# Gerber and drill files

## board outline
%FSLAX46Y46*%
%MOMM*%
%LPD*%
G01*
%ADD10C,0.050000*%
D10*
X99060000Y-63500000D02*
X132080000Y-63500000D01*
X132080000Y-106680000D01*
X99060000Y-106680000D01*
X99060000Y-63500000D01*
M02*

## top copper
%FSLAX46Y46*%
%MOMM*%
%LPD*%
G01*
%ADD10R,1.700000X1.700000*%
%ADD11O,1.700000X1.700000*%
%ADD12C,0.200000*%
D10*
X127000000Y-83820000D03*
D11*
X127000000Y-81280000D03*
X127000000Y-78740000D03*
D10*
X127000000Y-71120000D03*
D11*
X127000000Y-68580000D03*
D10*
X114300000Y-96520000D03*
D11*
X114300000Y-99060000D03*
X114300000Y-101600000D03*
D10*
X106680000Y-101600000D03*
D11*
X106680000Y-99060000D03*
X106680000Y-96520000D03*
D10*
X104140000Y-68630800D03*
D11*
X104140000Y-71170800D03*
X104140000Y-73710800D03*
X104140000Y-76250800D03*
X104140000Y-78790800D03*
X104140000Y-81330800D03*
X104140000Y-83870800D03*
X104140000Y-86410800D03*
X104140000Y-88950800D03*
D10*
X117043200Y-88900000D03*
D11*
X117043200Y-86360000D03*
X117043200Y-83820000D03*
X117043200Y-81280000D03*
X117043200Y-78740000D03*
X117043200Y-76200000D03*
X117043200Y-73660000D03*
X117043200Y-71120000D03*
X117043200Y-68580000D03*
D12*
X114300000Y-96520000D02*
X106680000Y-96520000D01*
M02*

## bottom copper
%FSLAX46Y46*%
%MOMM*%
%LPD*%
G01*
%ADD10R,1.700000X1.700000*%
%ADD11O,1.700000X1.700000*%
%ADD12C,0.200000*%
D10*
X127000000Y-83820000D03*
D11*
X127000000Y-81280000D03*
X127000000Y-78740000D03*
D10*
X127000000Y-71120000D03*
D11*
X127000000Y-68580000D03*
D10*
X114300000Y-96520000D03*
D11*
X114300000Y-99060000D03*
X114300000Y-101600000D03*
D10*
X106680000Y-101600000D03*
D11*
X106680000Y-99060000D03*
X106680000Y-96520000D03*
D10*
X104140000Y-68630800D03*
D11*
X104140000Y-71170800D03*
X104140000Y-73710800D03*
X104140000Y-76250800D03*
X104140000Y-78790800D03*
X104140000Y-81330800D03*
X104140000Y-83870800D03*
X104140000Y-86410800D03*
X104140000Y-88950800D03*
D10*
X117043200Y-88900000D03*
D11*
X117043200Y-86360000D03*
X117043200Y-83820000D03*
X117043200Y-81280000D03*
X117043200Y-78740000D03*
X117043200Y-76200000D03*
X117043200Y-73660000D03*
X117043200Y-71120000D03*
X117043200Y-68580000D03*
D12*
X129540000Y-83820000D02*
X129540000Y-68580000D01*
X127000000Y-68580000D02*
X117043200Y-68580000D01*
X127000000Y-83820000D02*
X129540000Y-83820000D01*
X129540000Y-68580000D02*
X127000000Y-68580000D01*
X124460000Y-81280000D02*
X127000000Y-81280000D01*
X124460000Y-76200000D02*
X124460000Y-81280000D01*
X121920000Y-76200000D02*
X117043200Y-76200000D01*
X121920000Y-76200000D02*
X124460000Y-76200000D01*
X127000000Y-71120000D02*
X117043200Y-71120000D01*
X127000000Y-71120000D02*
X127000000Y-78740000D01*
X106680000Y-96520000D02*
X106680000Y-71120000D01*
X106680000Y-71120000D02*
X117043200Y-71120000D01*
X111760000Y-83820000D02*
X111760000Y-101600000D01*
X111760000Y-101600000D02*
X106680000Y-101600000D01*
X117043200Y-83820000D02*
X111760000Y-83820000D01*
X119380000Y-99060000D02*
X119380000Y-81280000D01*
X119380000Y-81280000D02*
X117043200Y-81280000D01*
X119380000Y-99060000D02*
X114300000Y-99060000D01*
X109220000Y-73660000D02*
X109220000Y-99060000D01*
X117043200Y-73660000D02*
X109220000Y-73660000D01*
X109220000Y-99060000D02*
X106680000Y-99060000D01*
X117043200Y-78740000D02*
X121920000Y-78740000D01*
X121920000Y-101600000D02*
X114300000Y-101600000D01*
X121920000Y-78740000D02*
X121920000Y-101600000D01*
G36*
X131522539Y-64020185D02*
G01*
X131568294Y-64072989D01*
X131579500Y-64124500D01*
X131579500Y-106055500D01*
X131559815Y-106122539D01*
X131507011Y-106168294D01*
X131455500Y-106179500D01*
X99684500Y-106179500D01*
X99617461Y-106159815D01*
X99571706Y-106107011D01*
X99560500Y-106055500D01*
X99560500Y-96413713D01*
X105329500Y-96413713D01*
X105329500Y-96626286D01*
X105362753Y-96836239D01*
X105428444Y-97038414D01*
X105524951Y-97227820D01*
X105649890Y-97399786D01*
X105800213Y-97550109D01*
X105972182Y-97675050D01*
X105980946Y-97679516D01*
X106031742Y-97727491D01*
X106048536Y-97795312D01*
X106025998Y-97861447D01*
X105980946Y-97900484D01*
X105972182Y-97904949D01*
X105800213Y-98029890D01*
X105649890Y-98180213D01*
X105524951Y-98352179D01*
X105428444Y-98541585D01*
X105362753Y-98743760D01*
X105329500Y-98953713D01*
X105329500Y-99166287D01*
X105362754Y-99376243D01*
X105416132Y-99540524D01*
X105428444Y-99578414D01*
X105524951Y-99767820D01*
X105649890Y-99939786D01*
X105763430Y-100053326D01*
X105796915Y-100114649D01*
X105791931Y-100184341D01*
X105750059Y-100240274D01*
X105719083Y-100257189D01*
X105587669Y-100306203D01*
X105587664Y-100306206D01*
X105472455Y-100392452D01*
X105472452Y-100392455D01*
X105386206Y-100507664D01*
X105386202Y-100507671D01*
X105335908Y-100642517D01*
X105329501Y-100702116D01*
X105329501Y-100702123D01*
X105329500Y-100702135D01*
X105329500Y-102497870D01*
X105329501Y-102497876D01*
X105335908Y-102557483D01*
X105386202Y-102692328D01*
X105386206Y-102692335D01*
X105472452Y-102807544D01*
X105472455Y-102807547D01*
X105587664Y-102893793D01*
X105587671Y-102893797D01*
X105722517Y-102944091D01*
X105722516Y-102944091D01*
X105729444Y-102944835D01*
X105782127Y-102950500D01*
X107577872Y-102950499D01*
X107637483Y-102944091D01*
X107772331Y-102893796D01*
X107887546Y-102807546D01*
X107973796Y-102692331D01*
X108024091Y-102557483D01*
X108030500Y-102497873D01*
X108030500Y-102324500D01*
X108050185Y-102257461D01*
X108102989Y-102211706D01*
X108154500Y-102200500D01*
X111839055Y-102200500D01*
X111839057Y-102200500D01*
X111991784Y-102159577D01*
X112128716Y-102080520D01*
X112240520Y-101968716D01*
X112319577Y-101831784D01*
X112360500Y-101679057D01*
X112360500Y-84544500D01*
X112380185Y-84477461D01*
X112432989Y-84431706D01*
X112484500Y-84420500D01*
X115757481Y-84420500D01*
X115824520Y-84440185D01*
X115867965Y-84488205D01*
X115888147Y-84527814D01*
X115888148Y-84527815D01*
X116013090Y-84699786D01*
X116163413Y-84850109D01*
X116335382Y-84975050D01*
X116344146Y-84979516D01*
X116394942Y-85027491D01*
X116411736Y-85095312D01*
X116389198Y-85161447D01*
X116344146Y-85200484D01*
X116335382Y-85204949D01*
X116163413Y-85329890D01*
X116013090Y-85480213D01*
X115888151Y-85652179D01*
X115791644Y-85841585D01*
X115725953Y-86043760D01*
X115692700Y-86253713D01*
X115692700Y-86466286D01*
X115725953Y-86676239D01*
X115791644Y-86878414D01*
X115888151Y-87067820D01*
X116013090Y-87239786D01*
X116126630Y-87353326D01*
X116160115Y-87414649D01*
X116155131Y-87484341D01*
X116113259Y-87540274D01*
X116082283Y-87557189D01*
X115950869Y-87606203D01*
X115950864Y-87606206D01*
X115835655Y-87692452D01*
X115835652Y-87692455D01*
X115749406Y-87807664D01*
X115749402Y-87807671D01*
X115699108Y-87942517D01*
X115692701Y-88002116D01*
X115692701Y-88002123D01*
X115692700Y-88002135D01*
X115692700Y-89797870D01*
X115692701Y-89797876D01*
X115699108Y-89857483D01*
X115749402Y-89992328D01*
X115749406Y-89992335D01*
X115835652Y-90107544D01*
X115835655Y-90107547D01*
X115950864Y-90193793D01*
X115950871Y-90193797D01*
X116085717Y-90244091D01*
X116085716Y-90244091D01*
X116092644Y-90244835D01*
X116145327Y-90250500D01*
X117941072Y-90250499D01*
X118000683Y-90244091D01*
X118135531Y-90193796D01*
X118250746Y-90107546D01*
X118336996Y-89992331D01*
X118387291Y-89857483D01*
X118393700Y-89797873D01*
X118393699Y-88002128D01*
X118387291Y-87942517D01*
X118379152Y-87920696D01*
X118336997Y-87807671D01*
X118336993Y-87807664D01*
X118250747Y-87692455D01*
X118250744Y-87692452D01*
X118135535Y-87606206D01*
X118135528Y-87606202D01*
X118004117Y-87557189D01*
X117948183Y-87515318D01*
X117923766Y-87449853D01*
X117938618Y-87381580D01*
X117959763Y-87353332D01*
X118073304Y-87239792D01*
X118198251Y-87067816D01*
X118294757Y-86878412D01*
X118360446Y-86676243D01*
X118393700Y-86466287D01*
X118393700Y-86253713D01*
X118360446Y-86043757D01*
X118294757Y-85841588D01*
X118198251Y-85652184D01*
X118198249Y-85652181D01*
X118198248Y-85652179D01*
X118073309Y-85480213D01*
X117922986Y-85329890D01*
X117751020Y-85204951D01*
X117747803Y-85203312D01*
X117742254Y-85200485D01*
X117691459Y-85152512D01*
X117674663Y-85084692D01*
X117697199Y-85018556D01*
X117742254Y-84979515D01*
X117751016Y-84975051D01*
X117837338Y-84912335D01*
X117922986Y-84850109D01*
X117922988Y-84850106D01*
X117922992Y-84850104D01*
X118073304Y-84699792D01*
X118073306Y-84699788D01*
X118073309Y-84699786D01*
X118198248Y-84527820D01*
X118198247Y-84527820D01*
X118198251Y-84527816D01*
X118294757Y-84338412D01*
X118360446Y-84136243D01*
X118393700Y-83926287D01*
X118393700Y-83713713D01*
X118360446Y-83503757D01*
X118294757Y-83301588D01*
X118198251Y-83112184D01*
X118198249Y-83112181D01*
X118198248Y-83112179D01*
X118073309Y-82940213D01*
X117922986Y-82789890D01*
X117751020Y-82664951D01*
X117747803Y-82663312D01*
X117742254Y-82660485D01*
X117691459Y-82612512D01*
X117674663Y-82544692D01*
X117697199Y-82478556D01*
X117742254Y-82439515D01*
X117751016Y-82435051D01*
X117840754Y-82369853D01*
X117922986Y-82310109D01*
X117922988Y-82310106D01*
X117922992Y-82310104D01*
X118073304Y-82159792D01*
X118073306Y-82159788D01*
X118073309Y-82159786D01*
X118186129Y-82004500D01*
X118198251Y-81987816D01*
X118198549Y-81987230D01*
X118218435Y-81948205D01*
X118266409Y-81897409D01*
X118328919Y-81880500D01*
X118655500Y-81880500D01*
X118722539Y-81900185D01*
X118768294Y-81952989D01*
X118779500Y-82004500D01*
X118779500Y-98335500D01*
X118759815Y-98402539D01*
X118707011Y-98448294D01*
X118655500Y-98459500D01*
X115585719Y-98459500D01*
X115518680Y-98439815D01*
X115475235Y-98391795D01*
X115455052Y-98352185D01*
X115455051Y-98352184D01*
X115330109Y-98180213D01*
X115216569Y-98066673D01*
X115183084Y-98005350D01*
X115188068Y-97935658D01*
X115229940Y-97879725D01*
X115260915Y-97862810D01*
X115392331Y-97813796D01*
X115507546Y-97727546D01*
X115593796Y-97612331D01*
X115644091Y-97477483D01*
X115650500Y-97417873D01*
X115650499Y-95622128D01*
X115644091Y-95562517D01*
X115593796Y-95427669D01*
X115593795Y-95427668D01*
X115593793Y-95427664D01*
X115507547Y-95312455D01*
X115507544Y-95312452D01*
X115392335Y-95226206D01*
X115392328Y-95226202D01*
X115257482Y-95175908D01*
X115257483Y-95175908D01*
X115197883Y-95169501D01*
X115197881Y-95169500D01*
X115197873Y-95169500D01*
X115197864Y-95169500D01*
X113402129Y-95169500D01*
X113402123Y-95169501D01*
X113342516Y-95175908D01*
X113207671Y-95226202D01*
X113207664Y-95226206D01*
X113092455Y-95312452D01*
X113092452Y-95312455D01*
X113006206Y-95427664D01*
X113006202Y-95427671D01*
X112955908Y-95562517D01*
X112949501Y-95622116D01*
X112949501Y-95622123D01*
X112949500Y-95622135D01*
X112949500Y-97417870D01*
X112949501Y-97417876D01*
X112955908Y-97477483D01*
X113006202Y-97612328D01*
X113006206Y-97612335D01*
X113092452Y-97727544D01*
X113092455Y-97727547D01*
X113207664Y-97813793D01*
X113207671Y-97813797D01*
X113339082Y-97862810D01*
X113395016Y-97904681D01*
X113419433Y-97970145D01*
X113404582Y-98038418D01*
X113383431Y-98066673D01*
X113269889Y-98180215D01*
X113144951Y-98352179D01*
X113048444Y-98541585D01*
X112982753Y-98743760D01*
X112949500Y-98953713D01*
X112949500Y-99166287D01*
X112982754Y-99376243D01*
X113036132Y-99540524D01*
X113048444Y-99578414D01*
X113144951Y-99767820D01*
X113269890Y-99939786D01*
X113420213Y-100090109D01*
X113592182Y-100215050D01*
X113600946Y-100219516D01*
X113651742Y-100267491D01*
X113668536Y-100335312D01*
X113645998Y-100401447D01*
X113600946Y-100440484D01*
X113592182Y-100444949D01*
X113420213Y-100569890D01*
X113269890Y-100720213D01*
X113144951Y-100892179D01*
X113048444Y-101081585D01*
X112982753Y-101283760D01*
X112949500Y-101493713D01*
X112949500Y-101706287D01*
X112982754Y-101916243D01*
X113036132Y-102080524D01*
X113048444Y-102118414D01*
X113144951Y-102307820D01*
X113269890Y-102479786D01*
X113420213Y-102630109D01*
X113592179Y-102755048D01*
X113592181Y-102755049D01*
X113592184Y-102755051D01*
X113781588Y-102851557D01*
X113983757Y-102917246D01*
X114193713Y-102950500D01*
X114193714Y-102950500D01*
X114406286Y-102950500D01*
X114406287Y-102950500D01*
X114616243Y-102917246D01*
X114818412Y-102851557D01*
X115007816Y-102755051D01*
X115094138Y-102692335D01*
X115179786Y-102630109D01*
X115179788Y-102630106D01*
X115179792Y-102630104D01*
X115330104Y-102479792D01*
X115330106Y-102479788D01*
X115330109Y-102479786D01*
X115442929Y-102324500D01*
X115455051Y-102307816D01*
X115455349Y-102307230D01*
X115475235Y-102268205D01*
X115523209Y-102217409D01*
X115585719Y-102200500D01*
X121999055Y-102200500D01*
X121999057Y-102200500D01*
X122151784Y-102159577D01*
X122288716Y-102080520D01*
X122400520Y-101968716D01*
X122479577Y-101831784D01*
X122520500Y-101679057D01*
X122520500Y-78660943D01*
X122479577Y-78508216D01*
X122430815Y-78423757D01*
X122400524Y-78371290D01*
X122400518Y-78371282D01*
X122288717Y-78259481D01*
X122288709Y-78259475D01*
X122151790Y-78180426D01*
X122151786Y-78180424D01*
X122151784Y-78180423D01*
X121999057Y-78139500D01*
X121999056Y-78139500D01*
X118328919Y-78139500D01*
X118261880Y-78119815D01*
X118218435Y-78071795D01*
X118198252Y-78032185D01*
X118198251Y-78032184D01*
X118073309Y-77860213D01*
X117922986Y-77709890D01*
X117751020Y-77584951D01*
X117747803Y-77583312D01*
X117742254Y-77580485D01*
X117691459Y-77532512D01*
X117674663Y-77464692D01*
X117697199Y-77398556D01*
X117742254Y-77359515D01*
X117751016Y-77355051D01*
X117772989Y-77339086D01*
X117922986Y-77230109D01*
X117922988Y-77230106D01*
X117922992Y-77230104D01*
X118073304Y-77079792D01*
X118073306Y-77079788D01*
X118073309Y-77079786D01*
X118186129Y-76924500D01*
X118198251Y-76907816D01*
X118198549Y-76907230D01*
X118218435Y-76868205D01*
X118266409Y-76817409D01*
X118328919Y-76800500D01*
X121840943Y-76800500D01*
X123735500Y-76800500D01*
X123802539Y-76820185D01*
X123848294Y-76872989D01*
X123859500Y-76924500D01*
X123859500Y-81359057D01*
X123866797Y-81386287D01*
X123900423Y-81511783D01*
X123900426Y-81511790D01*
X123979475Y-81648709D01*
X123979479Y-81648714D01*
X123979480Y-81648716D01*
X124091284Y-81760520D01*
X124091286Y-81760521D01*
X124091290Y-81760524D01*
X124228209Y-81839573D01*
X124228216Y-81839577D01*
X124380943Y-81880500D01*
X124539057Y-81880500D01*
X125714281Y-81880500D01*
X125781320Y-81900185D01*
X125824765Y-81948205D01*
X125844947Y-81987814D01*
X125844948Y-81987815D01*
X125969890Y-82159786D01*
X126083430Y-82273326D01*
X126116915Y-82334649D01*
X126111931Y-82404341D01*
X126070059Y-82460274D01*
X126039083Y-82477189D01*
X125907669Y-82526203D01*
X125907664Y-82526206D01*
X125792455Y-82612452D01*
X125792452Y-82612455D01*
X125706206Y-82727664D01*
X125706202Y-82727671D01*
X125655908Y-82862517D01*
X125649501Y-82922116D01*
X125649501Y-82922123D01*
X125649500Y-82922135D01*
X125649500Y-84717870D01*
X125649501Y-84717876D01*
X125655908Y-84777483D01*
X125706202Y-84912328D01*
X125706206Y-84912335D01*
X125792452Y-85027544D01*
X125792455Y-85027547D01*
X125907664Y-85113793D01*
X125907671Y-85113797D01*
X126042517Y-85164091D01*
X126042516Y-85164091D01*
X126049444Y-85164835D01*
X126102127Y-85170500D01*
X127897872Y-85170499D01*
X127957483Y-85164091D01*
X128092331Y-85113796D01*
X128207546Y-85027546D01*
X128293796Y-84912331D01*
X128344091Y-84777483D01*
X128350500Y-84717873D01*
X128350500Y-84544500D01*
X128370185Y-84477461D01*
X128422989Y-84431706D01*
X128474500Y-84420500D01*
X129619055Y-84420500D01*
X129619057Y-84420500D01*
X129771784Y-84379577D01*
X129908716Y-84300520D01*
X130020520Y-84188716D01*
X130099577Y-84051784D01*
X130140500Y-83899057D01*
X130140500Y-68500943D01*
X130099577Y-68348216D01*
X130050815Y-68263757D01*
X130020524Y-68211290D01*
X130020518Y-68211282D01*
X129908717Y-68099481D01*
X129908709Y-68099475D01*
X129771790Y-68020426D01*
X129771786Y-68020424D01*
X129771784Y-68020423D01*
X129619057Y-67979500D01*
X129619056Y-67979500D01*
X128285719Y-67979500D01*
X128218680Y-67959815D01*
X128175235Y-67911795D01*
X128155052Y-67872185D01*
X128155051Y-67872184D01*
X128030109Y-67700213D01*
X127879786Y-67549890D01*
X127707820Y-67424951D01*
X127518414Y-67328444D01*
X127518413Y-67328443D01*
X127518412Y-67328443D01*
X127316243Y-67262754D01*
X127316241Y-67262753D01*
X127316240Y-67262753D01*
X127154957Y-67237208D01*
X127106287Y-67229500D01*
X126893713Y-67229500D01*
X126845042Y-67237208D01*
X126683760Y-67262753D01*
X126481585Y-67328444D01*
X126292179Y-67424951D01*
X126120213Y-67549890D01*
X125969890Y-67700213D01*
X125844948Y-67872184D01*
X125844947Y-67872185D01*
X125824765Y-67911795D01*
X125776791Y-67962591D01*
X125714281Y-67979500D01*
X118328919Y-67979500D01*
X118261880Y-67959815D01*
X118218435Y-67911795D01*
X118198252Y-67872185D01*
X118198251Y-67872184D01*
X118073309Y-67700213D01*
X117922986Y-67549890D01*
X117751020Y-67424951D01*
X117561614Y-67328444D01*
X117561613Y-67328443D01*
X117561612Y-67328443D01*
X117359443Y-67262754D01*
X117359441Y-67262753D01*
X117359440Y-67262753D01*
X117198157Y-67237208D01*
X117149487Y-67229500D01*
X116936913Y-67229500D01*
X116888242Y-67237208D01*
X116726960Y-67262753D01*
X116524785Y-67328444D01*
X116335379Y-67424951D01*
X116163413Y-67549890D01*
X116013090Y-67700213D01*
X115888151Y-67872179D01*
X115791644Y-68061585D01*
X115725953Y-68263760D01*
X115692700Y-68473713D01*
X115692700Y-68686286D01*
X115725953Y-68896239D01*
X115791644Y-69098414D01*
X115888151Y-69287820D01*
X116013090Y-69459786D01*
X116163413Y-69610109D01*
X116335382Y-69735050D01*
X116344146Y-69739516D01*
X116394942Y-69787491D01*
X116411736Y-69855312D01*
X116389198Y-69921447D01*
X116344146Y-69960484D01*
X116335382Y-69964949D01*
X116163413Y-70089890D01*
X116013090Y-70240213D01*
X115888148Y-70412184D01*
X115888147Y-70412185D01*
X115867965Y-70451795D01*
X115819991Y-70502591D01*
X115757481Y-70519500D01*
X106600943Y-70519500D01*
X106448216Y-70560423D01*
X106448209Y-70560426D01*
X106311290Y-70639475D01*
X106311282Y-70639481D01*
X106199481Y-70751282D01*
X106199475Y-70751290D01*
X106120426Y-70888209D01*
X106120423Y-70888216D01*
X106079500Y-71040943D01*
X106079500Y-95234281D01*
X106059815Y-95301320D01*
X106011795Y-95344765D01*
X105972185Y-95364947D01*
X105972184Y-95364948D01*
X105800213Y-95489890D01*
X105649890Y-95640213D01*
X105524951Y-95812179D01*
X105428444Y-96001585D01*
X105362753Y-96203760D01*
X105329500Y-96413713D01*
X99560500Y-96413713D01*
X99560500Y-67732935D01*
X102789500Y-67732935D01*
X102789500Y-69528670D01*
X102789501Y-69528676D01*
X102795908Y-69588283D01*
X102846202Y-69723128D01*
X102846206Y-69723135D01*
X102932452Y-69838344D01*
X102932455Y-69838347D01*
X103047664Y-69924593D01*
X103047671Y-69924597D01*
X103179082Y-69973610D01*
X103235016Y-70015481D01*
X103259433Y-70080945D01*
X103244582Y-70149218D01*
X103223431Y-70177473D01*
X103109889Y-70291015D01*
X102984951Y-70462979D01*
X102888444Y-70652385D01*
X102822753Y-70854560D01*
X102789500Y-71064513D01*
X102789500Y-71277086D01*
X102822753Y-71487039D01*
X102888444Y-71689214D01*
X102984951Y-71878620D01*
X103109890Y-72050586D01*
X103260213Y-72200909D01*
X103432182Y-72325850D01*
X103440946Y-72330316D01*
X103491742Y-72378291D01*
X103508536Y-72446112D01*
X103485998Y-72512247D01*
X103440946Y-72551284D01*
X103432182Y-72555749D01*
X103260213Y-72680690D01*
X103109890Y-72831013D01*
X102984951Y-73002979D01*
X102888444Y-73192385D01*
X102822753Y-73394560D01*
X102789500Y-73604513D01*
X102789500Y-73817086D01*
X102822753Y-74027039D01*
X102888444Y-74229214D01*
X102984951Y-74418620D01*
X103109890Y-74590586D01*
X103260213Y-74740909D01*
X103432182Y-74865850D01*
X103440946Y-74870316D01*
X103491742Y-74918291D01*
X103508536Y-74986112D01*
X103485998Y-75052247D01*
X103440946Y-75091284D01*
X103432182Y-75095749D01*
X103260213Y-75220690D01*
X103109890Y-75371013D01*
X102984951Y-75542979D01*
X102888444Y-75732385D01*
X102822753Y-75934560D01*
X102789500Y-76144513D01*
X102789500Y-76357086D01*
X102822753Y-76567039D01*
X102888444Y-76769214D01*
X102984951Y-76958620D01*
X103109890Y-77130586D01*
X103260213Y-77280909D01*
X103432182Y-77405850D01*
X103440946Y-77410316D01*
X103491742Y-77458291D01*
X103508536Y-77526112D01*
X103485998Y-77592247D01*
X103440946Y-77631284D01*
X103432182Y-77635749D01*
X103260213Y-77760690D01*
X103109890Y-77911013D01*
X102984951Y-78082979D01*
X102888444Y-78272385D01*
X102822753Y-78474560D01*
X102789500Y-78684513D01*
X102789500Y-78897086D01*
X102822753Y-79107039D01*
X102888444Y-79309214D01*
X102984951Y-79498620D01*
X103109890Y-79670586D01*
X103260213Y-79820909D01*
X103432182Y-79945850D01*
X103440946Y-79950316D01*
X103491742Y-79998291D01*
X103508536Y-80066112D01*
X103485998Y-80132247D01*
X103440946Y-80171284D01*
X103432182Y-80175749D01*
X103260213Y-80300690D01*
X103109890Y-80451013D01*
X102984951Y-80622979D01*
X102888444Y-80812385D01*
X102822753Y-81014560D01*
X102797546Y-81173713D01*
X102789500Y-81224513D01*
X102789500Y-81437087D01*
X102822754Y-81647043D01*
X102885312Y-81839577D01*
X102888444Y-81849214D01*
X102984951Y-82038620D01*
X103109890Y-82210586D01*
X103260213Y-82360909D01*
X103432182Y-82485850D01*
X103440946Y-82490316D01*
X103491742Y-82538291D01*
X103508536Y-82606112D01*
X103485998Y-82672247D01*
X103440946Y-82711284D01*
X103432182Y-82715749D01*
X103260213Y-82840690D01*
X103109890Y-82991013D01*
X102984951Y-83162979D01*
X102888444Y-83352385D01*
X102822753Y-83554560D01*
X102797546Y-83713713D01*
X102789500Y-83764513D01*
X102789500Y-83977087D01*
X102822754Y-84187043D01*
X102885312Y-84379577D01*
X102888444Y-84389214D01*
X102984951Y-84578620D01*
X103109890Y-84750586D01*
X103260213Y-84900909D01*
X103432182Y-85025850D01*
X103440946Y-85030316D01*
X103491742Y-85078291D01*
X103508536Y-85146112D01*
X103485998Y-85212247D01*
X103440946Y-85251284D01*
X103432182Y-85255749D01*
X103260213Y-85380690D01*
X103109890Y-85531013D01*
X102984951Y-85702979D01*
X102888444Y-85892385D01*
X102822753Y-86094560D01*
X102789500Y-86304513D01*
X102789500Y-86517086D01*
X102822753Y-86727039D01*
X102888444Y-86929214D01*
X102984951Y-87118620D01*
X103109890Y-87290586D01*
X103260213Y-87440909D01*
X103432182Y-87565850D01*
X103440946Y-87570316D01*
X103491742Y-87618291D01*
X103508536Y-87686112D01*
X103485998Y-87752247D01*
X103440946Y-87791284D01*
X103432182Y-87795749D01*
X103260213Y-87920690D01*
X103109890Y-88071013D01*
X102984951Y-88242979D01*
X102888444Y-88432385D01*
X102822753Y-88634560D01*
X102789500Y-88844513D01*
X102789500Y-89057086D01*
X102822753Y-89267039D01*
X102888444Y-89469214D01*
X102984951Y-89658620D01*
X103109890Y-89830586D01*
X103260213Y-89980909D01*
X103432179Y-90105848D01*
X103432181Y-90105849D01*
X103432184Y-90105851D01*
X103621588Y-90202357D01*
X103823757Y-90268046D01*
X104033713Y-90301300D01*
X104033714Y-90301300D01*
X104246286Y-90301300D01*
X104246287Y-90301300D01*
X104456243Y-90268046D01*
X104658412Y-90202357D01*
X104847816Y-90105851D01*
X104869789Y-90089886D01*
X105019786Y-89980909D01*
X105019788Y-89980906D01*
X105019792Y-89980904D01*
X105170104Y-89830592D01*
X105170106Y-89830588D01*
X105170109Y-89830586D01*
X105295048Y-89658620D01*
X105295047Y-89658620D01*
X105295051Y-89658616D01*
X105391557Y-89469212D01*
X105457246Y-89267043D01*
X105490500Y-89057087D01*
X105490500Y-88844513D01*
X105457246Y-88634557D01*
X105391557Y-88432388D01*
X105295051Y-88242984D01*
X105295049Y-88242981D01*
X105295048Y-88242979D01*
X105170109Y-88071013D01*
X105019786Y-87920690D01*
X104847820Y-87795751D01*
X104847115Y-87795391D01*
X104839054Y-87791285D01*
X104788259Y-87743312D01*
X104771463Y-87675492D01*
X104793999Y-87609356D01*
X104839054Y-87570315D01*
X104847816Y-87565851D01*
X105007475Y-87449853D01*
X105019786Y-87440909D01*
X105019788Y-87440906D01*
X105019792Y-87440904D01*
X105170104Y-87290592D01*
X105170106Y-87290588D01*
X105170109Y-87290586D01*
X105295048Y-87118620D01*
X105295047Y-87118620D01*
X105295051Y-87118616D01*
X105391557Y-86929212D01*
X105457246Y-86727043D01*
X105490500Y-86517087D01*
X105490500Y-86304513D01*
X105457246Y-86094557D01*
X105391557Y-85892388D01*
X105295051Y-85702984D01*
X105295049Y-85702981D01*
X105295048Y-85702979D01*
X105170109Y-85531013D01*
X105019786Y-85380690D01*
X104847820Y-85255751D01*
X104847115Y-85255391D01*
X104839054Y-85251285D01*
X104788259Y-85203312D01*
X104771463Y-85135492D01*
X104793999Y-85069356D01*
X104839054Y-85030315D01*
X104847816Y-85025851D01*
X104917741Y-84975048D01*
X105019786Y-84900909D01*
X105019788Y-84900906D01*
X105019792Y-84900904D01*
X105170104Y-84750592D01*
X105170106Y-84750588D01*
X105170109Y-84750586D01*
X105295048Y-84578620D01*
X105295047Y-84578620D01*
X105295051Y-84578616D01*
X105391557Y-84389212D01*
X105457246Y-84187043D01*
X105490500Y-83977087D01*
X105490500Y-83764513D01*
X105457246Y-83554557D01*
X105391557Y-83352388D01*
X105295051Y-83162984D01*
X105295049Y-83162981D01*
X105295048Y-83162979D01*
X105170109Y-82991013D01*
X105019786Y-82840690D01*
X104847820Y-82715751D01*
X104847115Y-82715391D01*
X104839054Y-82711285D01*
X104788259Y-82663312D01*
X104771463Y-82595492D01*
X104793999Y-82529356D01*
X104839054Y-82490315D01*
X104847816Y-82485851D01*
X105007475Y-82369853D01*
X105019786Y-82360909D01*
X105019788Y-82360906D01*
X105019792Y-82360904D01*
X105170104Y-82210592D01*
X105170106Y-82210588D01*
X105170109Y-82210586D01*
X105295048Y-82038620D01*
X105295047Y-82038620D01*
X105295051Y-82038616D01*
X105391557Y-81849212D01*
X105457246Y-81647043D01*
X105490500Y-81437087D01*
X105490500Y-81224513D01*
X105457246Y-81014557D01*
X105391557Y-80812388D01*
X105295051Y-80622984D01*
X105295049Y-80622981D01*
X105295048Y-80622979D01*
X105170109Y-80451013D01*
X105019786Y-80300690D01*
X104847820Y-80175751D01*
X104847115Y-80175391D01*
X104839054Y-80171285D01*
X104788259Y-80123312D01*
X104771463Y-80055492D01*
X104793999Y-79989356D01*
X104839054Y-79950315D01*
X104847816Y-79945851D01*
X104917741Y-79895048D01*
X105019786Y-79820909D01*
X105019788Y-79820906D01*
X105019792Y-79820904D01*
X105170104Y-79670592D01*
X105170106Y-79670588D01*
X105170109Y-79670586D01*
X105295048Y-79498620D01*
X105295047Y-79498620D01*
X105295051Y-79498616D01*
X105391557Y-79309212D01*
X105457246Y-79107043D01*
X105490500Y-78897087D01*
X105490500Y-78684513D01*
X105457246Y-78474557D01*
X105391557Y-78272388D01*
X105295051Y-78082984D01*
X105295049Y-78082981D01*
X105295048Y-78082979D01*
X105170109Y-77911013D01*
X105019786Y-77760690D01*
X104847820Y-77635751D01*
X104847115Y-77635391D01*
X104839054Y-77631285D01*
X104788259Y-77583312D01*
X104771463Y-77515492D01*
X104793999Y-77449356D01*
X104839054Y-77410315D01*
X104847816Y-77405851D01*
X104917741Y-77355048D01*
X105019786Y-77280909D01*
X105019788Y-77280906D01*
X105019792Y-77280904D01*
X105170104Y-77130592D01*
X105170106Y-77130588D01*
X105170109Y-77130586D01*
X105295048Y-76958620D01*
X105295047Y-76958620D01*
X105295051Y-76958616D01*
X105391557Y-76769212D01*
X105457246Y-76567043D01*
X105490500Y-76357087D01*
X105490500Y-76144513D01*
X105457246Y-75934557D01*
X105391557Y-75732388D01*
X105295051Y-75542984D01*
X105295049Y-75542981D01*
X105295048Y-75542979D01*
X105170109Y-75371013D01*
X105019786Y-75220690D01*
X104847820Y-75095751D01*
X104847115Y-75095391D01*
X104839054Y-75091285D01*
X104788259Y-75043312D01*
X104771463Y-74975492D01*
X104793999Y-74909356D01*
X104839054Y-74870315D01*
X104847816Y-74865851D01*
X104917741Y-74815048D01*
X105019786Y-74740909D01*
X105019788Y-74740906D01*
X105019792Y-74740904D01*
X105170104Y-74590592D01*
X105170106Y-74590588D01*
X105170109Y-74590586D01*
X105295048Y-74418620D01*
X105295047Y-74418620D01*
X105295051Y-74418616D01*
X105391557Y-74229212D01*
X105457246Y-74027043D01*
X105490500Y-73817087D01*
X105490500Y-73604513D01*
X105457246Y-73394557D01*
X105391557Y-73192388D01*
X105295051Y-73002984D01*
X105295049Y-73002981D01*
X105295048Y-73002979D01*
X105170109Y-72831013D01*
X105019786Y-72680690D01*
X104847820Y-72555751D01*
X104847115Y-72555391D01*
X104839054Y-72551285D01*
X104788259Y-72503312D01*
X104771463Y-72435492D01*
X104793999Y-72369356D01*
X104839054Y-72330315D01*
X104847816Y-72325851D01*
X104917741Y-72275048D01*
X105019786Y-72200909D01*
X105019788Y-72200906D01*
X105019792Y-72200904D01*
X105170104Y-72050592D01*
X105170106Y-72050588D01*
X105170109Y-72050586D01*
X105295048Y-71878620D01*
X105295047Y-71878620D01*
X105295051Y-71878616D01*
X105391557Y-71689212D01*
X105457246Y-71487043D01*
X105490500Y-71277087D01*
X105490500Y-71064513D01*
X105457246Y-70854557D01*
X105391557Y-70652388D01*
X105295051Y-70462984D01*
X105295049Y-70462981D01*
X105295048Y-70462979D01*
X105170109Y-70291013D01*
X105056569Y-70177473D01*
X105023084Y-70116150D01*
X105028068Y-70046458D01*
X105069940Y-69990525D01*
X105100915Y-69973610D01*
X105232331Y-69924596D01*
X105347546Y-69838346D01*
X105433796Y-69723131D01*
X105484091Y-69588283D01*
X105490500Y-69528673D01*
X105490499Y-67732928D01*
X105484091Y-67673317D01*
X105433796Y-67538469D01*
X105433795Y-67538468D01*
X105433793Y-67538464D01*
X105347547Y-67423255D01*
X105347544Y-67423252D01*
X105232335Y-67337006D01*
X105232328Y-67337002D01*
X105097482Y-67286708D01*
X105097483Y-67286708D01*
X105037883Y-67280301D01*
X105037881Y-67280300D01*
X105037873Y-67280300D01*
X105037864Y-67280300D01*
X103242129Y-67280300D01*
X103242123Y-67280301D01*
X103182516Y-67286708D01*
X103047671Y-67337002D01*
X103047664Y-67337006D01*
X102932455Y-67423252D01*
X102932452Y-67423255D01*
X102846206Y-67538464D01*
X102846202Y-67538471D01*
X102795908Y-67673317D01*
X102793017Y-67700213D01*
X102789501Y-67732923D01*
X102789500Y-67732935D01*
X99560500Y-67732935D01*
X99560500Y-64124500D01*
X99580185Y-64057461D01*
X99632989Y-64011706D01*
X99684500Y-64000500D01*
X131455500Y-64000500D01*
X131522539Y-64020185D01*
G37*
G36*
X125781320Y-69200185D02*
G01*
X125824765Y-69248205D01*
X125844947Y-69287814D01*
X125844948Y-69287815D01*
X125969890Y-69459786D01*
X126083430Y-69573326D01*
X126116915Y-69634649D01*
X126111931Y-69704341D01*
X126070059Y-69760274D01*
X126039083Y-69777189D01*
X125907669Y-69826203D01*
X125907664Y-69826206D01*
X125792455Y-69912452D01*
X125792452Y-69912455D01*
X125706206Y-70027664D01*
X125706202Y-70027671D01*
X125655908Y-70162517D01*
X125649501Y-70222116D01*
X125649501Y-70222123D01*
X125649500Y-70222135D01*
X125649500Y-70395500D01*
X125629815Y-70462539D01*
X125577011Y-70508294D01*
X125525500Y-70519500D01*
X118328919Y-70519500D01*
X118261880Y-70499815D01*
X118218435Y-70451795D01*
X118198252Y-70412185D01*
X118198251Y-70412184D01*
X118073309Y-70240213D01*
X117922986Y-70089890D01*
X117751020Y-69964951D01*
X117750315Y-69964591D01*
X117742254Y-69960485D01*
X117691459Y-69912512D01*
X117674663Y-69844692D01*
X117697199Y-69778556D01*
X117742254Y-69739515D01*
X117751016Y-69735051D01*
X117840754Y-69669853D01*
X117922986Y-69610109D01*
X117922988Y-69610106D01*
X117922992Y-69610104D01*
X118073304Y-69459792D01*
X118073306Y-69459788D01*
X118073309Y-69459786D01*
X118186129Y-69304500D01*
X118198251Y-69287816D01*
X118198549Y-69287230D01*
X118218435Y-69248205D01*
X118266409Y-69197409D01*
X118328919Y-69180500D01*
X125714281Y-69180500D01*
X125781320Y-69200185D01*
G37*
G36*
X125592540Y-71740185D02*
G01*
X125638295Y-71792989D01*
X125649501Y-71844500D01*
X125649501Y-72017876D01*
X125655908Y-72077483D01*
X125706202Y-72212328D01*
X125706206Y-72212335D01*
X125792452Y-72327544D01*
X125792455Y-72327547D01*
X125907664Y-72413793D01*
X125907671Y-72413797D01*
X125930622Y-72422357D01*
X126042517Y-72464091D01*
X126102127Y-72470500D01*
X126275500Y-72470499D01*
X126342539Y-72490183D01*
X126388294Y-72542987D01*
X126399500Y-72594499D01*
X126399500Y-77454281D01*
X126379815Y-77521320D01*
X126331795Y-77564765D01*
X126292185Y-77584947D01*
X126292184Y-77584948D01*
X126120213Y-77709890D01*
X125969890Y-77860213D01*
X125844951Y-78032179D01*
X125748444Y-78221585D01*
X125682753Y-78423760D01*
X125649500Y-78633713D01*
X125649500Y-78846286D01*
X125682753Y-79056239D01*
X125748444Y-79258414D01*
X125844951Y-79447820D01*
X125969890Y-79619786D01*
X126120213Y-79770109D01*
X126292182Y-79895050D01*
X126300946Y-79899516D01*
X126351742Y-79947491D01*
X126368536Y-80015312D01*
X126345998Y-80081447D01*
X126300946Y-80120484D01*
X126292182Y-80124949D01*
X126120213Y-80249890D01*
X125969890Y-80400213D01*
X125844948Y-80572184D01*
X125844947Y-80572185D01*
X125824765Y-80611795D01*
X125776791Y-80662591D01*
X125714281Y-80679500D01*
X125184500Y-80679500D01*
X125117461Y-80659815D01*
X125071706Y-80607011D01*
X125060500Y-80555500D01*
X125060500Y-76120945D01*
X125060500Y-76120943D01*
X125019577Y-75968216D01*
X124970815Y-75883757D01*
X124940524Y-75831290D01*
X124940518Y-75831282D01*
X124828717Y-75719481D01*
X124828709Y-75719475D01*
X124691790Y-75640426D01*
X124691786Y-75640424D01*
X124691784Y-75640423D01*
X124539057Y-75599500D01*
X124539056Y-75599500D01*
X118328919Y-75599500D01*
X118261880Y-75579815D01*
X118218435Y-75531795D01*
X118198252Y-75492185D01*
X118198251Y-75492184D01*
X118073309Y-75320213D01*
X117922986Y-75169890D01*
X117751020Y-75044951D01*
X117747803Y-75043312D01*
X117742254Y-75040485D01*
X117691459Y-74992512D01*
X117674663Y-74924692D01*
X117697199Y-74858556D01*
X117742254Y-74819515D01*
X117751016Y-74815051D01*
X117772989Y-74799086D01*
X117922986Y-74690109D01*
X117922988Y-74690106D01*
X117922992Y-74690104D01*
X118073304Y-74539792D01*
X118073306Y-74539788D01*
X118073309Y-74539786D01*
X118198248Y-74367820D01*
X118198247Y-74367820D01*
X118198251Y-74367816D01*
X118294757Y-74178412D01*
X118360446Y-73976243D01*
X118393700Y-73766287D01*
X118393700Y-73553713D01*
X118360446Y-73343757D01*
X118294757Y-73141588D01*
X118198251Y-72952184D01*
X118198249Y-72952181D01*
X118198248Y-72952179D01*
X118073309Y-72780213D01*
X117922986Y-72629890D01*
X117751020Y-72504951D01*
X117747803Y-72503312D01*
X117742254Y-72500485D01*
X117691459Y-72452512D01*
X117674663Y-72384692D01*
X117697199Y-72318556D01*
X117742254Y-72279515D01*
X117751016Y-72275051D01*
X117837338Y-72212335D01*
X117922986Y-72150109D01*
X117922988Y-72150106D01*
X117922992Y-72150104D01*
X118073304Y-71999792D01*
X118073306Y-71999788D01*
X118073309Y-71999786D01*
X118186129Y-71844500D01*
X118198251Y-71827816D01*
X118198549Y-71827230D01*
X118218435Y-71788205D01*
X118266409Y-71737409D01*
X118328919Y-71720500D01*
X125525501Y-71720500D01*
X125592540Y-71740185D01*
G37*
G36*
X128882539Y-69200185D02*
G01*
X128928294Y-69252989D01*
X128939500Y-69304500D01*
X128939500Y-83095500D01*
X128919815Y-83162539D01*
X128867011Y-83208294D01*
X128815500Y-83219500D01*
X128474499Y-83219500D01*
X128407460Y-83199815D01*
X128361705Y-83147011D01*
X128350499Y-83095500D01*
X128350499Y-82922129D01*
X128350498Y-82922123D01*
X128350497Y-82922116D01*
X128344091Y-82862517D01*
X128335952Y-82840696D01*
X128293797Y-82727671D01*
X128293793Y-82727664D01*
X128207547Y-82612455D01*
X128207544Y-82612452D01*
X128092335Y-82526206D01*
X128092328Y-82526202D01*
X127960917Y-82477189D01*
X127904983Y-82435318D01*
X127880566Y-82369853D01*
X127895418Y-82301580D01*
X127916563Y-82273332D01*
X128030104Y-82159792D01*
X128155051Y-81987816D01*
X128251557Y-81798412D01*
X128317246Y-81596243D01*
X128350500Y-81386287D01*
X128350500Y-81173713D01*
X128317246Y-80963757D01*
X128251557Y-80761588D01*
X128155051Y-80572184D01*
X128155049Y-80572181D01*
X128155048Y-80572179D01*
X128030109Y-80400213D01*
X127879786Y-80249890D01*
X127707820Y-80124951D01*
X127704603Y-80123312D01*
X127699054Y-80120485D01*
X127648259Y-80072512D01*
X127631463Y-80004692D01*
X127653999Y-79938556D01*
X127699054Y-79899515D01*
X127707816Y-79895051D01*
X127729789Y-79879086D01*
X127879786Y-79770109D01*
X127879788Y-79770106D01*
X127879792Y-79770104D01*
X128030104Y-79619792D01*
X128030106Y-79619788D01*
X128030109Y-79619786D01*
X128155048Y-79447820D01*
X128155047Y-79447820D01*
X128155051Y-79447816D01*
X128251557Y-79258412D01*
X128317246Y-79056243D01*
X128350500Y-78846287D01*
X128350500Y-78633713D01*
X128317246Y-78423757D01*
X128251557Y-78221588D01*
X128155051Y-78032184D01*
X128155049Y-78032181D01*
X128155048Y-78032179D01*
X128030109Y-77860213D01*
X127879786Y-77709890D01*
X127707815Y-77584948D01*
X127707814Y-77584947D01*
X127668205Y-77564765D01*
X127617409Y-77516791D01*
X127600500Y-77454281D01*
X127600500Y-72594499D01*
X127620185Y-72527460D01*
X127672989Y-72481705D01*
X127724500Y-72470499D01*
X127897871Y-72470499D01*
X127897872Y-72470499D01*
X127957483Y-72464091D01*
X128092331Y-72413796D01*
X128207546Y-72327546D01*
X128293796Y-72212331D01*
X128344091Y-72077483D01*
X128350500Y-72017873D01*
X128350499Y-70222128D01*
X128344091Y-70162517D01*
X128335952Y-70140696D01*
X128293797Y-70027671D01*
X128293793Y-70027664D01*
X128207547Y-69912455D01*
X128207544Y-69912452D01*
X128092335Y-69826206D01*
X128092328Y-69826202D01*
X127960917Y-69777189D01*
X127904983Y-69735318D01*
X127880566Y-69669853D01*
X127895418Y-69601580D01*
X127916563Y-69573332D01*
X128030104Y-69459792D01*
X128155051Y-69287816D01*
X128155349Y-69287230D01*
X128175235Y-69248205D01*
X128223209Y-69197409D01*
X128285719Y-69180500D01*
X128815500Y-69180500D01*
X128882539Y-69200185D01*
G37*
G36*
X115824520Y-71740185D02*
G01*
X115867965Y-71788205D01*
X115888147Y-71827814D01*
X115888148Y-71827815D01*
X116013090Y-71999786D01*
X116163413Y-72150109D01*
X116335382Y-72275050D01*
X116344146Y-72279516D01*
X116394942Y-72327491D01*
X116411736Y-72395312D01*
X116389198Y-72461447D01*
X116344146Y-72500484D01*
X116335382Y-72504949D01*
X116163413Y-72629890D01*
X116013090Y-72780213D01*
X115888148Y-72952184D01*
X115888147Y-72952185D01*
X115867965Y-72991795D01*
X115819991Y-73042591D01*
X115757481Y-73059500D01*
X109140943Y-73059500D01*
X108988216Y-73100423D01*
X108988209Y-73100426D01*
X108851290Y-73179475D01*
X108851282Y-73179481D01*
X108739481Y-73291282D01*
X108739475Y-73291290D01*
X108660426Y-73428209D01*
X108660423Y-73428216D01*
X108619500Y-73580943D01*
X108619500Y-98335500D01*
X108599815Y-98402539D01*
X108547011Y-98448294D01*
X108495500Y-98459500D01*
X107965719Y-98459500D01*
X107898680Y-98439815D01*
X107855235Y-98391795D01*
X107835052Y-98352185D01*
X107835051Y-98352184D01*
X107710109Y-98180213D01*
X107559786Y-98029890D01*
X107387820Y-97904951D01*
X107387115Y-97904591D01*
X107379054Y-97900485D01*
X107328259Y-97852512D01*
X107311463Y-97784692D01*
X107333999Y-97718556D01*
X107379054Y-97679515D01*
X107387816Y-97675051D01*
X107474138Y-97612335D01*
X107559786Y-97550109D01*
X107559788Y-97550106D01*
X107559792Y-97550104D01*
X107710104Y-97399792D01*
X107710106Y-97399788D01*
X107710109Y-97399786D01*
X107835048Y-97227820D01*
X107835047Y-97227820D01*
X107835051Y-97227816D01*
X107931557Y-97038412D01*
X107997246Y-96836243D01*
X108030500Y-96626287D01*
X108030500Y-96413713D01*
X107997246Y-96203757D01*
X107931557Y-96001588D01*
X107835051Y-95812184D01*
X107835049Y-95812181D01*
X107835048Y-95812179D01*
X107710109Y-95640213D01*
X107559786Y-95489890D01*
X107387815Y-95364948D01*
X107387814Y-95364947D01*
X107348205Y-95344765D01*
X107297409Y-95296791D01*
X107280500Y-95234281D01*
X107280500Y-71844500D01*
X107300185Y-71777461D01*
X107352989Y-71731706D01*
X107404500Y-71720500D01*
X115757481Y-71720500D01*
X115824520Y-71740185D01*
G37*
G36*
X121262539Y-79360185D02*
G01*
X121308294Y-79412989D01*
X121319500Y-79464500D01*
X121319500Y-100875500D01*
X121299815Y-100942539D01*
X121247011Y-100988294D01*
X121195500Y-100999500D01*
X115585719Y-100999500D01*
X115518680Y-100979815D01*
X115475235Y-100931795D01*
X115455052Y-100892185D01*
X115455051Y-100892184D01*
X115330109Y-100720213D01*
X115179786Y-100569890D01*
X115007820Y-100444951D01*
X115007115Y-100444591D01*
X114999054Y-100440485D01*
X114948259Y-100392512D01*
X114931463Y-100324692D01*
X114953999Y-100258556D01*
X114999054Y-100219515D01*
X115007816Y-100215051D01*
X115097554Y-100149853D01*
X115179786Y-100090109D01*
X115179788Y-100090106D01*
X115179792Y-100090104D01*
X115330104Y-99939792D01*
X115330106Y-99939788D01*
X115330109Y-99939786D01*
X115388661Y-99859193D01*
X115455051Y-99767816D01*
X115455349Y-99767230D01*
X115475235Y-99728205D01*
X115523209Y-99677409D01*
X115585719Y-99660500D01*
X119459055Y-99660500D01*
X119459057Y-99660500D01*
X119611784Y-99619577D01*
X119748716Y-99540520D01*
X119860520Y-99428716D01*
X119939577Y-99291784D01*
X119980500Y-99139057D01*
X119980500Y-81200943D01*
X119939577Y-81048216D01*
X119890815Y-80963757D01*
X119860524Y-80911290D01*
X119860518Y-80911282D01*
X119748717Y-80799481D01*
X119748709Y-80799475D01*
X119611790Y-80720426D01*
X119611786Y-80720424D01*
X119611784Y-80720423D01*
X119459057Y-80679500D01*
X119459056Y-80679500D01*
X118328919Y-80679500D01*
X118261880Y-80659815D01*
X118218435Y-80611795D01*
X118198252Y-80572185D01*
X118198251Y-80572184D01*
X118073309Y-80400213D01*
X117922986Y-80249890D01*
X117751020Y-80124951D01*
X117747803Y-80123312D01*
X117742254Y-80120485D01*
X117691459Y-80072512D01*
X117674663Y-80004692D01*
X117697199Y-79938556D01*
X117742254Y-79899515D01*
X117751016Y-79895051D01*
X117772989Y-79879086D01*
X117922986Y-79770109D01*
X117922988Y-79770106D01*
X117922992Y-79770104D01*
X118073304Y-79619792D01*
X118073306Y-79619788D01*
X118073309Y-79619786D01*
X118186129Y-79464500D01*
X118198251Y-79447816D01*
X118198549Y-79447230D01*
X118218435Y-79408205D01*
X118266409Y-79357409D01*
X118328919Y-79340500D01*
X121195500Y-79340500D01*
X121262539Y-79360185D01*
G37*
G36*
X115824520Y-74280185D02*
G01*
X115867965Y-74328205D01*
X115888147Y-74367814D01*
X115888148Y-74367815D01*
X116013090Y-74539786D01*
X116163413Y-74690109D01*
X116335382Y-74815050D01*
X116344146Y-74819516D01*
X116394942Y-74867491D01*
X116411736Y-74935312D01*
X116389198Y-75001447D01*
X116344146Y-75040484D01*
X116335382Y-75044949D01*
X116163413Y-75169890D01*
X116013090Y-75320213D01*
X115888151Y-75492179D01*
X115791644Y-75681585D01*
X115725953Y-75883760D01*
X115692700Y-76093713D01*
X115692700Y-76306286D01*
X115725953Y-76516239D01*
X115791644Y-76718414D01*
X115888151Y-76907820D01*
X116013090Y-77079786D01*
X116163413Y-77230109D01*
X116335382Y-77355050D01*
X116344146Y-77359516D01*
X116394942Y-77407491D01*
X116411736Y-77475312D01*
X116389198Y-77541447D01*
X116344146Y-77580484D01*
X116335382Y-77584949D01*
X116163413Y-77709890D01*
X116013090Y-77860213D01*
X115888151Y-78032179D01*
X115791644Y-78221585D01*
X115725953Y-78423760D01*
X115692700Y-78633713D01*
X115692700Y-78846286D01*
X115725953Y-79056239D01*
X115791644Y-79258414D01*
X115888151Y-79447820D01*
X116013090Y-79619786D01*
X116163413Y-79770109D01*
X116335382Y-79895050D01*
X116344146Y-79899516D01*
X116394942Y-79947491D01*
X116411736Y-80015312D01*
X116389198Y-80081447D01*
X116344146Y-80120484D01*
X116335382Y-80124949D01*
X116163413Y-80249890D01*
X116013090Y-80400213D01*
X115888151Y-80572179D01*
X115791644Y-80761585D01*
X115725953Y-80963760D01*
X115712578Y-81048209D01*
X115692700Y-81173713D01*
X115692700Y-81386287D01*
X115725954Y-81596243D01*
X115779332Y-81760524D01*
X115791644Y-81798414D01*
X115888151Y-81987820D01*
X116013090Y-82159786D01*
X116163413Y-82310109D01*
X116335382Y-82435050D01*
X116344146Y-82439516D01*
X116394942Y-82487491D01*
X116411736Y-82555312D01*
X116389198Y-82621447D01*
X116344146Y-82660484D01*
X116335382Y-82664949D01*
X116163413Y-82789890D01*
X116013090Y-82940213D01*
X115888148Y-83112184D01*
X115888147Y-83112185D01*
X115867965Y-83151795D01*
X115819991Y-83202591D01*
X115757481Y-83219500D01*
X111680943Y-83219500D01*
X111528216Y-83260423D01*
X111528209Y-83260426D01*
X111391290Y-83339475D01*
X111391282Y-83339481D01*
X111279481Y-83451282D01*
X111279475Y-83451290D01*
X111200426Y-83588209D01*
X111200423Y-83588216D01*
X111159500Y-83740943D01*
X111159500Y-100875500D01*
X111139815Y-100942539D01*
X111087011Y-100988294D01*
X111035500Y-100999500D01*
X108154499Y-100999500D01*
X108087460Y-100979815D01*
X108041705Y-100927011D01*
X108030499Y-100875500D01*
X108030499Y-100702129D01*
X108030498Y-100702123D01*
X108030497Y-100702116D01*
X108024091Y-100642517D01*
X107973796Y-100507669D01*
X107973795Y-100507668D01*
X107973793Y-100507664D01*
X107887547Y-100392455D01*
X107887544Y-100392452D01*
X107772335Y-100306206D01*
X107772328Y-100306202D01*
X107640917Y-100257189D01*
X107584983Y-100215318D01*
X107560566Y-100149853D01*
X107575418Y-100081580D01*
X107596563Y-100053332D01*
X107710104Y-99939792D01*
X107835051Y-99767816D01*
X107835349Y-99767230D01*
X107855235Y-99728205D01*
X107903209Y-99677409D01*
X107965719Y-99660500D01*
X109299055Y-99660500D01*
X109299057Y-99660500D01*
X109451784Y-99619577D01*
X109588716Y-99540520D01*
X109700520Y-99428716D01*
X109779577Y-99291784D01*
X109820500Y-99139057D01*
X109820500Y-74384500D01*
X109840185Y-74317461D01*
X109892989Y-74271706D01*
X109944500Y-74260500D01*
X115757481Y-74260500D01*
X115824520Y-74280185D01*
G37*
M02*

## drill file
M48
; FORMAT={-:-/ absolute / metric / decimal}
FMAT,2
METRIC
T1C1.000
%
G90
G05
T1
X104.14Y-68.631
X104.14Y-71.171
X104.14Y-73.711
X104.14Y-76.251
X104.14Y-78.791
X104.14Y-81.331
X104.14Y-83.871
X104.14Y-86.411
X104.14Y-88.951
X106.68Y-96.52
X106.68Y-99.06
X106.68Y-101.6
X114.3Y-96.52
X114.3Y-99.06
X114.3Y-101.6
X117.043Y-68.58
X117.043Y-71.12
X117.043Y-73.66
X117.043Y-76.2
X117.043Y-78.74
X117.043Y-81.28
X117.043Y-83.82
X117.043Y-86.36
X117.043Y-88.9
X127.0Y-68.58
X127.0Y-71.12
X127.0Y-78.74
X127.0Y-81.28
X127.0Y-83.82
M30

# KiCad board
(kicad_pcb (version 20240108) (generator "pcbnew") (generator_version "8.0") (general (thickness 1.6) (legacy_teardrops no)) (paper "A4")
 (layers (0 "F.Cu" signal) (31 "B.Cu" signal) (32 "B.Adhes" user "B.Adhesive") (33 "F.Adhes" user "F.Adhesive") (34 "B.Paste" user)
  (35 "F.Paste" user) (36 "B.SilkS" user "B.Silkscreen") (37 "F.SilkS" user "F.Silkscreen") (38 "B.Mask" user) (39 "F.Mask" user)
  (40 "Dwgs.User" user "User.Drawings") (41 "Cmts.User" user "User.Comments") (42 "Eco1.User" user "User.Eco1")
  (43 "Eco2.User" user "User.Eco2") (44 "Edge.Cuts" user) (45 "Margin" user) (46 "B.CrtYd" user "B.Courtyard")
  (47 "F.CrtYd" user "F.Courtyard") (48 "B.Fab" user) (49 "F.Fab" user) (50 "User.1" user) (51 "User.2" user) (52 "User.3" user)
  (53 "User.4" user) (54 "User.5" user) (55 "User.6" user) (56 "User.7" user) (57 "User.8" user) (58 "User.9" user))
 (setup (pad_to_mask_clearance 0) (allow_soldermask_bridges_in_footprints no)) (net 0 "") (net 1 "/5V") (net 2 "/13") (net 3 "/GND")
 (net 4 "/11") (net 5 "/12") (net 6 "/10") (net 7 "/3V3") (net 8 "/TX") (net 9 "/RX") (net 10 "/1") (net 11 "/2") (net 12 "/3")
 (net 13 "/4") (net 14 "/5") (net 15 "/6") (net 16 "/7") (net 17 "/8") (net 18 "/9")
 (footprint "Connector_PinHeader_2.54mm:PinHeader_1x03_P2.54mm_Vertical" (layer "F.Cu") (at 127 83.82 180)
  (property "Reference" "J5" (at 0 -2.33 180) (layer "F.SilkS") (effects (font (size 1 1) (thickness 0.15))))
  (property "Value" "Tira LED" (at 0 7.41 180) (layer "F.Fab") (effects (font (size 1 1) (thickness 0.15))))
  (pad "1" thru_hole rect (at 0 0 180) (size 1.7 1.7) (drill 1) (layers "*.Cu" "*.Mask") (remove_unused_layers no) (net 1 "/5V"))
  (pad "2" thru_hole oval (at 0 2.54 180) (size 1.7 1.7) (drill 1) (layers "*.Cu" "*.Mask") (remove_unused_layers no) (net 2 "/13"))
  (pad "3" thru_hole oval (at 0 5.08 180) (size 1.7 1.7) (drill 1) (layers "*.Cu" "*.Mask") (remove_unused_layers no) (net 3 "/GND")))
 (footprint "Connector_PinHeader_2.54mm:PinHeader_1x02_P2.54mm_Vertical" (layer "F.Cu") (at 127 71.12 180)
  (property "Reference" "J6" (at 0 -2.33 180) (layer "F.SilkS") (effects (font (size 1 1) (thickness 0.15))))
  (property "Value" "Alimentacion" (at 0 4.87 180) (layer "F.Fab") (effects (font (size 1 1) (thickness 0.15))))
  (pad "1" thru_hole rect (at 0 0 180) (size 1.7 1.7) (drill 1) (layers "*.Cu" "*.Mask") (remove_unused_layers no) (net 3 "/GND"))
  (pad "2" thru_hole oval (at 0 2.54 180) (size 1.7 1.7) (drill 1) (layers "*.Cu" "*.Mask") (remove_unused_layers no) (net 1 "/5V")))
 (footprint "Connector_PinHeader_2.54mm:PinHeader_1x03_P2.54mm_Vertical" (layer "F.Cu") (at 114.3 96.52)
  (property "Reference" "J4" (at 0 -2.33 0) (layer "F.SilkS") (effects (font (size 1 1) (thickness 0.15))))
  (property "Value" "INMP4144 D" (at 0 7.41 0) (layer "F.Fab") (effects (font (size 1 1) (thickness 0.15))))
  (pad "1" thru_hole rect (at 0 0) (size 1.7 1.7) (drill 1) (layers "*.Cu" "*.Mask") (remove_unused_layers no) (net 3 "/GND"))
  (pad "2" thru_hole oval (at 0 2.54) (size 1.7 1.7) (drill 1) (layers "*.Cu" "*.Mask") (remove_unused_layers no) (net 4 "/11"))
  (pad "3" thru_hole oval (at 0 5.08) (size 1.7 1.7) (drill 1) (layers "*.Cu" "*.Mask") (remove_unused_layers no) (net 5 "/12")))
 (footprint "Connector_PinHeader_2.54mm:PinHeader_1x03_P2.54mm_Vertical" (layer "F.Cu") (at 106.68 101.6 180)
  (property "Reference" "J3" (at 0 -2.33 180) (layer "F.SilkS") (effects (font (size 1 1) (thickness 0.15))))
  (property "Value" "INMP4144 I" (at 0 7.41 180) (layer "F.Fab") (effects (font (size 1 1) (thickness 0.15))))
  (pad "1" thru_hole rect (at 0 0 180) (size 1.7 1.7) (drill 1) (layers "*.Cu" "*.Mask") (remove_unused_layers no) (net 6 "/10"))
  (pad "2" thru_hole oval (at 0 2.54 180) (size 1.7 1.7) (drill 1) (layers "*.Cu" "*.Mask") (remove_unused_layers no) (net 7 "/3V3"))
  (pad "3" thru_hole oval (at 0 5.08 180) (size 1.7 1.7) (drill 1) (layers "*.Cu" "*.Mask") (remove_unused_layers no) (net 3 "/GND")))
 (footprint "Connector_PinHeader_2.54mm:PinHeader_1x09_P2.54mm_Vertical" (layer "F.Cu") (at 104.14 68.6308)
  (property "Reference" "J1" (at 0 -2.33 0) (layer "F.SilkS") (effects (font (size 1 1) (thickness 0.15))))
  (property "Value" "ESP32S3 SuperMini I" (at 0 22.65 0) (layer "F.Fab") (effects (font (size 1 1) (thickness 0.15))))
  (pad "1" thru_hole rect (at 0 0) (size 1.7 1.7) (drill 1) (layers "*.Cu" "*.Mask") (remove_unused_layers no) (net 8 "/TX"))
  (pad "2" thru_hole oval (at 0 2.54) (size 1.7 1.7) (drill 1) (layers "*.Cu" "*.Mask") (remove_unused_layers no) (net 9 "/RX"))
  (pad "3" thru_hole oval (at 0 5.08) (size 1.7 1.7) (drill 1) (layers "*.Cu" "*.Mask") (remove_unused_layers no) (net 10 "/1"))
  (pad "4" thru_hole oval (at 0 7.62) (size 1.7 1.7) (drill 1) (layers "*.Cu" "*.Mask") (remove_unused_layers no) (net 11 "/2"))
  (pad "5" thru_hole oval (at 0 10.16) (size 1.7 1.7) (drill 1) (layers "*.Cu" "*.Mask") (remove_unused_layers no) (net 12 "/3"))
  (pad "6" thru_hole oval (at 0 12.7) (size 1.7 1.7) (drill 1) (layers "*.Cu" "*.Mask") (remove_unused_layers no) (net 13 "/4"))
  (pad "7" thru_hole oval (at 0 15.24) (size 1.7 1.7) (drill 1) (layers "*.Cu" "*.Mask") (remove_unused_layers no) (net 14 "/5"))
  (pad "8" thru_hole oval (at 0 17.78) (size 1.7 1.7) (drill 1) (layers "*.Cu" "*.Mask") (remove_unused_layers no) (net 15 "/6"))
  (pad "9" thru_hole oval (at 0 20.32) (size 1.7 1.7) (drill 1) (layers "*.Cu" "*.Mask") (remove_unused_layers no) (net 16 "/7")))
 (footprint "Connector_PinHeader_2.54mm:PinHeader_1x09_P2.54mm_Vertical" (layer "F.Cu") (at 117.0432 88.9 180)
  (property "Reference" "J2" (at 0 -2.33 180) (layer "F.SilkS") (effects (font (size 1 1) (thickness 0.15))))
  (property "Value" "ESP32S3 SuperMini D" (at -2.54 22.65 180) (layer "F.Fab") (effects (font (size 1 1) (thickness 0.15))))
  (pad "1" thru_hole rect (at 0 0 180) (size 1.7 1.7) (drill 1) (layers "*.Cu" "*.Mask") (remove_unused_layers no) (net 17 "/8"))
  (pad "2" thru_hole oval (at 0 2.54 180) (size 1.7 1.7) (drill 1) (layers "*.Cu" "*.Mask") (remove_unused_layers no) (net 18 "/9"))
  (pad "3" thru_hole oval (at 0 5.08 180) (size 1.7 1.7) (drill 1) (layers "*.Cu" "*.Mask") (remove_unused_layers no) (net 6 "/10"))
  (pad "4" thru_hole oval (at 0 7.62 180) (size 1.7 1.7) (drill 1) (layers "*.Cu" "*.Mask") (remove_unused_layers no) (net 4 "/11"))
  (pad "5" thru_hole oval (at 0 10.16 180) (size 1.7 1.7) (drill 1) (layers "*.Cu" "*.Mask") (remove_unused_layers no) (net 5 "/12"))
  (pad "6" thru_hole oval (at 0 12.7 180) (size 1.7 1.7) (drill 1) (layers "*.Cu" "*.Mask") (remove_unused_layers no) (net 2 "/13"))
  (pad "7" thru_hole oval (at 0 15.24 180) (size 1.7 1.7) (drill 1) (layers "*.Cu" "*.Mask") (remove_unused_layers no) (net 7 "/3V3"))
  (pad "8" thru_hole oval (at 0 17.78 180) (size 1.7 1.7) (drill 1) (layers "*.Cu" "*.Mask") (remove_unused_layers no) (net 3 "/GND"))
  (pad "9" thru_hole oval (at 0 20.32 180) (size 1.7 1.7) (drill 1) (layers "*.Cu" "*.Mask") (remove_unused_layers no) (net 1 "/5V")))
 (gr_rect (start 99.06 63.5) (end 132.08 106.68) (stroke (width 0.05) (type default)) (fill none) (layer "Edge.Cuts"))
 (segment (start 129.54 83.82) (end 129.54 68.58) (width 0.2) (layer "B.Cu") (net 1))
 (segment (start 127 68.58) (end 117.0432 68.58) (width 0.2) (layer "B.Cu") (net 1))
 (segment (start 127 83.82) (end 129.54 83.82) (width 0.2) (layer "B.Cu") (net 1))
 (segment (start 129.54 68.58) (end 127 68.58) (width 0.2) (layer "B.Cu") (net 1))
 (segment (start 124.46 81.28) (end 127 81.28) (width 0.2) (layer "B.Cu") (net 2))
 (segment (start 124.46 76.2) (end 124.46 81.28) (width 0.2) (layer "B.Cu") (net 2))
 (segment (start 121.92 76.2) (end 117.0432 76.2) (width 0.2) (layer "B.Cu") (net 2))
 (segment (start 121.92 76.2) (end 124.46 76.2) (width 0.2) (layer "B.Cu") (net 2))
 (segment (start 114.3 96.52) (end 106.68 96.52) (width 0.2) (layer "F.Cu") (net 3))
 (segment (start 127 71.12) (end 117.0432 71.12) (width 0.2) (layer "B.Cu") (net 3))
 (segment (start 127 71.12) (end 127 78.74) (width 0.2) (layer "B.Cu") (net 3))
 (segment (start 106.68 96.52) (end 106.68 71.12) (width 0.2) (layer "B.Cu") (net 3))
 (segment (start 106.68 71.12) (end 117.0432 71.12) (width 0.2) (layer "B.Cu") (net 3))
 (segment (start 111.76 83.82) (end 111.76 101.6) (width 0.2) (layer "B.Cu") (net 6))
 (segment (start 111.76 101.6) (end 106.68 101.6) (width 0.2) (layer "B.Cu") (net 6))
 (segment (start 117.0432 83.82) (end 111.76 83.82) (width 0.2) (layer "B.Cu") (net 6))
 (segment (start 119.38 99.06) (end 119.38 81.28) (width 0.2) (layer "B.Cu") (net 4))
 (segment (start 119.38 81.28) (end 117.0432 81.28) (width 0.2) (layer "B.Cu") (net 4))
 (segment (start 119.38 99.06) (end 114.3 99.06) (width 0.2) (layer "B.Cu") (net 4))
 (segment (start 109.22 73.66) (end 109.22 99.06) (width 0.2) (layer "B.Cu") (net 7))
 (segment (start 117.0432 73.66) (end 109.22 73.66) (width 0.2) (layer "B.Cu") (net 7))
 (segment (start 109.22 99.06) (end 106.68 99.06) (width 0.2) (layer "B.Cu") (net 7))
 (segment (start 117.0432 78.74) (end 121.92 78.74) (width 0.2) (layer "B.Cu") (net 5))
 (segment (start 121.92 101.6) (end 114.3 101.6) (width 0.2) (layer "B.Cu") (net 5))
 (segment (start 121.92 78.74) (end 121.92 101.6) (width 0.2) (layer "B.Cu") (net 5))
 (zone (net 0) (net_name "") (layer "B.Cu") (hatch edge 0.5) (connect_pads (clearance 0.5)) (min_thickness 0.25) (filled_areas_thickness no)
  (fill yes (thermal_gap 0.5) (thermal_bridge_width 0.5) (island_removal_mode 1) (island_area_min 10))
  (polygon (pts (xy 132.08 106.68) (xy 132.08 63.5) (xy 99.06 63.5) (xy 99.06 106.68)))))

